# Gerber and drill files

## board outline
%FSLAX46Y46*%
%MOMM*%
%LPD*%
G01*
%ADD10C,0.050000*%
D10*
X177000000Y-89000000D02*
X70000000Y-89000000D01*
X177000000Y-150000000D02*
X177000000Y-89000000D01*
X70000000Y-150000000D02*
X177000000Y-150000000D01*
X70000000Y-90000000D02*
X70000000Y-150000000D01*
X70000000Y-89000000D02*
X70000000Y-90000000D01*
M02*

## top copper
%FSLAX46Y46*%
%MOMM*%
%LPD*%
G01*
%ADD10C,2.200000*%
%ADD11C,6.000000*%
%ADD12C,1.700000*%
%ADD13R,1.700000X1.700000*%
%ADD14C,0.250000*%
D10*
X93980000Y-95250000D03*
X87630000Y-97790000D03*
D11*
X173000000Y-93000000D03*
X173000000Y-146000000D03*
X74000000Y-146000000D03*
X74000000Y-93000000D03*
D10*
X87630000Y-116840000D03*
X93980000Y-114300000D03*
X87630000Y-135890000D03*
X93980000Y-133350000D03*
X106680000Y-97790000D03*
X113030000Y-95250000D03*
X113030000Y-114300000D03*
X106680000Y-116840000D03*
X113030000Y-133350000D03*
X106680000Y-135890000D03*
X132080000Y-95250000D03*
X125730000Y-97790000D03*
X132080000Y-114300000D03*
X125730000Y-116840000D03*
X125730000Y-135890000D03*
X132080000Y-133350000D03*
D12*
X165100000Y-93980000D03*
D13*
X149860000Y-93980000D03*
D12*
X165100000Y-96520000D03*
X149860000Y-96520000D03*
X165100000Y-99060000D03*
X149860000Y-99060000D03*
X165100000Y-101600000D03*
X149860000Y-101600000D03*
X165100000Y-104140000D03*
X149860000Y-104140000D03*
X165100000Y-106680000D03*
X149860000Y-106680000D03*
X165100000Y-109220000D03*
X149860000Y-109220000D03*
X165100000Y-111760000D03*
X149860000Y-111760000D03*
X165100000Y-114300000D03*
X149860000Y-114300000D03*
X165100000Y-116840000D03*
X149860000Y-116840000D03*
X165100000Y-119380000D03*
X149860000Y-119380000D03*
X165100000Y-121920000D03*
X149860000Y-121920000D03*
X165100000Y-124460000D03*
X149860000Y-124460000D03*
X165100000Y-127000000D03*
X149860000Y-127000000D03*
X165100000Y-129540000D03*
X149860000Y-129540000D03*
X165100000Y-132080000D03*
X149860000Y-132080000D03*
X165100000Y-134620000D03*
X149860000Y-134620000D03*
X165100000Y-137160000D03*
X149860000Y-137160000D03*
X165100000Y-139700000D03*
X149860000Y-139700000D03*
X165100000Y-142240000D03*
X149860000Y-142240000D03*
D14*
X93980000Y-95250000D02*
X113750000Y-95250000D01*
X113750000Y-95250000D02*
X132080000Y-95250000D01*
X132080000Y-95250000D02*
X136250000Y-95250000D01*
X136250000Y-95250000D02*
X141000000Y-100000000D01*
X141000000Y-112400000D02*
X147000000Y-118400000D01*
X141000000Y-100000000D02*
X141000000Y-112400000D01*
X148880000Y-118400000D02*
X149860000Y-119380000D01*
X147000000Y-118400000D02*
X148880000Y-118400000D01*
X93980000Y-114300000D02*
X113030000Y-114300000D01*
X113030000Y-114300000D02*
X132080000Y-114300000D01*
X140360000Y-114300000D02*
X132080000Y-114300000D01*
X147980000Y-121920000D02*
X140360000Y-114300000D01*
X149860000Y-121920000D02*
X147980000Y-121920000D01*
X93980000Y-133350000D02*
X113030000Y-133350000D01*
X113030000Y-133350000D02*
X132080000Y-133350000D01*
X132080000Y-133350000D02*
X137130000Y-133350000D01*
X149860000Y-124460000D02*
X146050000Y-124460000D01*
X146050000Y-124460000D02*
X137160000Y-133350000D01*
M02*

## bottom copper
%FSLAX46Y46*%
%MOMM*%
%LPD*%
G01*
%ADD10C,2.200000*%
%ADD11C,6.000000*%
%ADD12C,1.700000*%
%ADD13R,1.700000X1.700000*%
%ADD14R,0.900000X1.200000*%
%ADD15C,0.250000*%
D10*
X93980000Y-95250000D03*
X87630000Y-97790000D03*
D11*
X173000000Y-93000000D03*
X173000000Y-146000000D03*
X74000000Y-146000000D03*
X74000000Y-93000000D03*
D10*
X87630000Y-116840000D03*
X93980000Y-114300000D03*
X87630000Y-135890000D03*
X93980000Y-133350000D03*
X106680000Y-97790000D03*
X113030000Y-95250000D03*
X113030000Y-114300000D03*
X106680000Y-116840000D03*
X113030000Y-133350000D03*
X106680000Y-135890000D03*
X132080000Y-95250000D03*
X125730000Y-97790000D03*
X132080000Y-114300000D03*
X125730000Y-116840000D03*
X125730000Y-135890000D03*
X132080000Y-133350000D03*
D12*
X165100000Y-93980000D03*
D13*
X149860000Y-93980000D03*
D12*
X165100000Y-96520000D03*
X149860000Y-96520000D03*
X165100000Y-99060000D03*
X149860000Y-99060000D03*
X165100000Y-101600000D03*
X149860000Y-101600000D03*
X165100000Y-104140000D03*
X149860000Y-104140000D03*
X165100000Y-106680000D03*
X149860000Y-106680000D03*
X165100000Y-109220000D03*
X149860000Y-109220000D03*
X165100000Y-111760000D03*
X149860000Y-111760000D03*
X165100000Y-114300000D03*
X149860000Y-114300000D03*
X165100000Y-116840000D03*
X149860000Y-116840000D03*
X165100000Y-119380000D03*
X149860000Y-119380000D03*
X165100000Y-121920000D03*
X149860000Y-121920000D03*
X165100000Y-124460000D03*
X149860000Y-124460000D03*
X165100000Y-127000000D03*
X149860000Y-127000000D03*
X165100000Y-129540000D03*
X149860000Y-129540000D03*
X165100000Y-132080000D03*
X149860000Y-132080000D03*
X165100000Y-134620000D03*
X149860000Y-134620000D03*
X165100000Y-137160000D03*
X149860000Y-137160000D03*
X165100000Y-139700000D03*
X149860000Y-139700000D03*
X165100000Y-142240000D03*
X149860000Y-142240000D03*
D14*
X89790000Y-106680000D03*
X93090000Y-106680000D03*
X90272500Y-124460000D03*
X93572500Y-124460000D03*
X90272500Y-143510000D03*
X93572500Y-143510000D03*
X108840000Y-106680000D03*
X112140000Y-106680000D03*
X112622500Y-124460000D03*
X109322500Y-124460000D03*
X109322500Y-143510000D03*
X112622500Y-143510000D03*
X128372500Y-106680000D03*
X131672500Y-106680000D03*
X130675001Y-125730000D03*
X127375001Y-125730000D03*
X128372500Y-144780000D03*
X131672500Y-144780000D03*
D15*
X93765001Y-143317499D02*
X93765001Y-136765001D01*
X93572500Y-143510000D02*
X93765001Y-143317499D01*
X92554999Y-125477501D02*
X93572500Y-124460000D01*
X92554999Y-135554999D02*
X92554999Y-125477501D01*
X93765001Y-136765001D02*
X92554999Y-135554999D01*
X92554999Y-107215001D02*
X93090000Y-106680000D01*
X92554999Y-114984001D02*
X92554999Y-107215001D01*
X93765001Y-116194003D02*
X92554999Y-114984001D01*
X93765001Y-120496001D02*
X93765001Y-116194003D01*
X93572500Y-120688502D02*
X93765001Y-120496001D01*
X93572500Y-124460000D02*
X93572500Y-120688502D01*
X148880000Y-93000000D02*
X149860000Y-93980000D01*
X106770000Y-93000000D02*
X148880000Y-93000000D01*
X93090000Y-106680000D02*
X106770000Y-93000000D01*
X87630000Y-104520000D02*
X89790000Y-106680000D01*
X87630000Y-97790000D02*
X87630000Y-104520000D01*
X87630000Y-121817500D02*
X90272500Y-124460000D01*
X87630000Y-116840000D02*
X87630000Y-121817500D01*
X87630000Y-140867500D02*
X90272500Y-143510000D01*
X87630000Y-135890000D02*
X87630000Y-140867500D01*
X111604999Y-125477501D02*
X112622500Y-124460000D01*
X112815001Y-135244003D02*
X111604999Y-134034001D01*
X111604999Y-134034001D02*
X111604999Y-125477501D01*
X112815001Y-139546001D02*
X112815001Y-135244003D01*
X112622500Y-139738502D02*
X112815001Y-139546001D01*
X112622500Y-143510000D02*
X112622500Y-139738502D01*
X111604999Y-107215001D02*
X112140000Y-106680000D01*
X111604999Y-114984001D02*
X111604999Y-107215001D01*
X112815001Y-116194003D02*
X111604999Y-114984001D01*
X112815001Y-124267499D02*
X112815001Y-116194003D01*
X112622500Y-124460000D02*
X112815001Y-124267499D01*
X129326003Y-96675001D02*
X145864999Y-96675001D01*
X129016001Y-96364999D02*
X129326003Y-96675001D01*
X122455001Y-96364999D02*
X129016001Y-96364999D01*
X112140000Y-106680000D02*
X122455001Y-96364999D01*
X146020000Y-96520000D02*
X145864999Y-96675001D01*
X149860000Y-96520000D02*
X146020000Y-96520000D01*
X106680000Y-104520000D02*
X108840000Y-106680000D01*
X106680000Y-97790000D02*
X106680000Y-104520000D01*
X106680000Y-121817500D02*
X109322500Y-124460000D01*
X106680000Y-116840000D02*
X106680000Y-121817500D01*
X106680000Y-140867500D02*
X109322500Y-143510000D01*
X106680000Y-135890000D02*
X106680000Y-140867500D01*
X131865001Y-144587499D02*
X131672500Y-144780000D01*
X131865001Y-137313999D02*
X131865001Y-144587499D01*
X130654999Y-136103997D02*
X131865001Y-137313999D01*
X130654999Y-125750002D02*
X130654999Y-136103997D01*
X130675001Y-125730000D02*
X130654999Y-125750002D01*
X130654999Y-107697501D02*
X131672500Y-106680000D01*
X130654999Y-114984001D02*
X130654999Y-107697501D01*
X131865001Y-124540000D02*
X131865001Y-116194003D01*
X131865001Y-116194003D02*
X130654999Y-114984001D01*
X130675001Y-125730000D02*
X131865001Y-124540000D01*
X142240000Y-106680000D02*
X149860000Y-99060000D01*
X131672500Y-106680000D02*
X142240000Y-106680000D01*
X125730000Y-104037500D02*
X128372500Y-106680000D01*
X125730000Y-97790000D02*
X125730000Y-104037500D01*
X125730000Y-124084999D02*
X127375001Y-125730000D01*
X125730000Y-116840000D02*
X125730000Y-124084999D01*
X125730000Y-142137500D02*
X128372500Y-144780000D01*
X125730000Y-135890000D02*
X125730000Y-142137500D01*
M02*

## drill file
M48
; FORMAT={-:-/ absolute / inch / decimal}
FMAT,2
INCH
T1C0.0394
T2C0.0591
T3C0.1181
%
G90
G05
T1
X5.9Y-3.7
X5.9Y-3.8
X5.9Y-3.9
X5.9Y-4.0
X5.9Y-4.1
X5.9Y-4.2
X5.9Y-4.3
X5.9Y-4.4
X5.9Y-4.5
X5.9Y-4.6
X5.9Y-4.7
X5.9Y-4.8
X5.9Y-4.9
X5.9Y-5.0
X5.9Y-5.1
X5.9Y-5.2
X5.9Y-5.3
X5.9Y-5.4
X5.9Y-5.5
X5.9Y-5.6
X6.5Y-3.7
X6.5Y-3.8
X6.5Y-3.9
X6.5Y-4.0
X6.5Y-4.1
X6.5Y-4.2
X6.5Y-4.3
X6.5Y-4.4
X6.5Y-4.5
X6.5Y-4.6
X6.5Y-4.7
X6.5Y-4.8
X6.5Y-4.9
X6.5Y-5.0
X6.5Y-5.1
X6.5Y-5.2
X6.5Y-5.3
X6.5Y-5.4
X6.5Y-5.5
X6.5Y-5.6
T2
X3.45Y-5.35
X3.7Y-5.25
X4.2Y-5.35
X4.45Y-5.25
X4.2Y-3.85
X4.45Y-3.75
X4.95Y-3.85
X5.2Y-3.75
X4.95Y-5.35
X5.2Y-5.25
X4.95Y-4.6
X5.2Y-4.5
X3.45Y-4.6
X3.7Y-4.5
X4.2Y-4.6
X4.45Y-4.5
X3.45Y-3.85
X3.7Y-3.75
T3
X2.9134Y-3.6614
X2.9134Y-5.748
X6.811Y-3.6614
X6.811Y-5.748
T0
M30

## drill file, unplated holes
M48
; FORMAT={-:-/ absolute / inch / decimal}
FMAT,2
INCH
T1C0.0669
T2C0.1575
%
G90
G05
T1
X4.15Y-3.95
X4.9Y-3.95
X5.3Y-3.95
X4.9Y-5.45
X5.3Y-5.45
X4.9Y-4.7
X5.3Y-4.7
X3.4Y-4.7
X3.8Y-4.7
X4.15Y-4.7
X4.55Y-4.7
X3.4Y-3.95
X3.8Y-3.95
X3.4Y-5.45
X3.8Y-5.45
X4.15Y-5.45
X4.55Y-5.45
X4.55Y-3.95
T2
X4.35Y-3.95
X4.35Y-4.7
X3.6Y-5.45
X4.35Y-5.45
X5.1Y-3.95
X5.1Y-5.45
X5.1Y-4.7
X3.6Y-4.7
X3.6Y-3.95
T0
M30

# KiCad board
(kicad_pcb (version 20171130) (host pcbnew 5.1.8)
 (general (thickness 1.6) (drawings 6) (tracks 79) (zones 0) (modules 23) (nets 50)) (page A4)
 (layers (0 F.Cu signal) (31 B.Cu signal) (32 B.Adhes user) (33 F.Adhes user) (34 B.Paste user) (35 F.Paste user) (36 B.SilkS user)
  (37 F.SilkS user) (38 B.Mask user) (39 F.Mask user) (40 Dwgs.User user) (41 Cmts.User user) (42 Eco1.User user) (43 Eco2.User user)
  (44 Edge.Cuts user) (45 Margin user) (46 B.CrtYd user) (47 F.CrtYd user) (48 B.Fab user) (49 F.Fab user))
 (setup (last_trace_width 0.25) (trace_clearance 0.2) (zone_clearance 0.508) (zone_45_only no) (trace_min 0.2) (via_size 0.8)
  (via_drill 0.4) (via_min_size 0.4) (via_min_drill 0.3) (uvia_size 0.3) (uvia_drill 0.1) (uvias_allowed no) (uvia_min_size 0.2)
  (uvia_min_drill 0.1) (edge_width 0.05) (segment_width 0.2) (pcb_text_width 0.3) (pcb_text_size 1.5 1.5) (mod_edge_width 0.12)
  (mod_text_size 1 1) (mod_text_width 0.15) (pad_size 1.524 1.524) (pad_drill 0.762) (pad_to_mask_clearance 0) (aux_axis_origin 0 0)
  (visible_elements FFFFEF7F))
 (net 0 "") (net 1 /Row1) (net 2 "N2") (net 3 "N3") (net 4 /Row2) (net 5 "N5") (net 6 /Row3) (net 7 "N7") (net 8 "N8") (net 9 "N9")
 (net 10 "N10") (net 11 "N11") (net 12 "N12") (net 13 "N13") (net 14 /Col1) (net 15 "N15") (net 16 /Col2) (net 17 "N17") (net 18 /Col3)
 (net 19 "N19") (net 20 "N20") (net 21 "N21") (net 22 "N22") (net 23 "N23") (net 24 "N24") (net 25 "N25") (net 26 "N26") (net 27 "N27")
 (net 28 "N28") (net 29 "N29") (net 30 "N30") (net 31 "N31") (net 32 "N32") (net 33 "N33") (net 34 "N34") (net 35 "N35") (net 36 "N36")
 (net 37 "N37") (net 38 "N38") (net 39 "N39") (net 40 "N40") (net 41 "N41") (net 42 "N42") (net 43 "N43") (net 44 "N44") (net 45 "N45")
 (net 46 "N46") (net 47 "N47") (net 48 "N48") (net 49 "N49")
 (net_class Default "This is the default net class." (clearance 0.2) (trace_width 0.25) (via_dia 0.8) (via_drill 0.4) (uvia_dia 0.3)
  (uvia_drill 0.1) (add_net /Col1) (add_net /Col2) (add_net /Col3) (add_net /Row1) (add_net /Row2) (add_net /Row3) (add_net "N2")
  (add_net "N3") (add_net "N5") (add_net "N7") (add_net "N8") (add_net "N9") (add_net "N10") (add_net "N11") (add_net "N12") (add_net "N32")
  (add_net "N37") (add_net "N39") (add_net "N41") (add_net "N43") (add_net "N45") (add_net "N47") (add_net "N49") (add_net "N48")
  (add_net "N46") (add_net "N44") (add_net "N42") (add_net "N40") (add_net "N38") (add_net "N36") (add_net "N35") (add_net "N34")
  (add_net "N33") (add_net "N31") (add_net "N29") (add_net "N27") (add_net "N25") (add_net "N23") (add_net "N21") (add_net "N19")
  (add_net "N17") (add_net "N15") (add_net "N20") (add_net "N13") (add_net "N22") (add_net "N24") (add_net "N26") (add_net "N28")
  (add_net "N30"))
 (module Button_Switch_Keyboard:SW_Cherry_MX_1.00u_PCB (layer F.Cu) (at 93.98 95.25)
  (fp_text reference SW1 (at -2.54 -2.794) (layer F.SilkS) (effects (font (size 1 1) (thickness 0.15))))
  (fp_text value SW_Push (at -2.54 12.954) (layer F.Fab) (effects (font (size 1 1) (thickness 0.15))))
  (pad 1 thru_hole circle (at 0 0) (size 2.2 2.2) (drill 1.5) (layers *.Cu *.Mask) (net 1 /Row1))
  (pad 2 thru_hole circle (at -6.35 2.54) (size 2.2 2.2) (drill 1.5) (layers *.Cu *.Mask) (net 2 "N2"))
  (pad "" np_thru_hole circle (at -2.54 5.08) (size 4 4) (drill 4) (layers *.Cu *.Mask))
  (pad "" np_thru_hole circle (at -7.62 5.08) (size 1.7 1.7) (drill 1.7) (layers *.Cu *.Mask))
  (pad "" np_thru_hole circle (at 2.54 5.08) (size 1.7 1.7) (drill 1.7) (layers *.Cu *.Mask)))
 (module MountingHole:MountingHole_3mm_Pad (layer F.Cu) (at 173 93)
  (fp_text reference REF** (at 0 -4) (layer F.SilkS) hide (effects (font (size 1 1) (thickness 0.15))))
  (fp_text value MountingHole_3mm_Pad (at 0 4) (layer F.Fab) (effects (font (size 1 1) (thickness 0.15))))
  (pad 1 thru_hole circle (at 0 0) (size 6 6) (drill 3) (layers *.Cu *.Mask)))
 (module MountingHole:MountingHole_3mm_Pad (layer F.Cu) (at 173 146)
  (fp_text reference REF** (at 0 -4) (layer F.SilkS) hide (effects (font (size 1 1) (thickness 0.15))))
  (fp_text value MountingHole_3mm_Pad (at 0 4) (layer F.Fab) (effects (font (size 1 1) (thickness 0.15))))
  (pad 1 thru_hole circle (at 0 0) (size 6 6) (drill 3) (layers *.Cu *.Mask)))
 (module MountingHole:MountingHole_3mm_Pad (layer F.Cu) (at 74 146)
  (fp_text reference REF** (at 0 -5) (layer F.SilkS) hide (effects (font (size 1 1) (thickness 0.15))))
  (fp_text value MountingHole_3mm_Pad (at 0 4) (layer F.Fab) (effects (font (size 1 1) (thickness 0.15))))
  (pad 1 thru_hole circle (at 0 0) (size 6 6) (drill 3) (layers *.Cu *.Mask)))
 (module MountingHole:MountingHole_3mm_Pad (layer F.Cu) (at 74 93)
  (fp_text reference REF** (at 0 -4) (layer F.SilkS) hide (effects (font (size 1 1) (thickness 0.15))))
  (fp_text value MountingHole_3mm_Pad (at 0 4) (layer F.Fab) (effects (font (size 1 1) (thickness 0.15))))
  (pad 1 thru_hole circle (at 0 0) (size 6 6) (drill 3) (layers *.Cu *.Mask)))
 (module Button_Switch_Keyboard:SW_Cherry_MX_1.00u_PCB (layer F.Cu) (at 93.98 114.3)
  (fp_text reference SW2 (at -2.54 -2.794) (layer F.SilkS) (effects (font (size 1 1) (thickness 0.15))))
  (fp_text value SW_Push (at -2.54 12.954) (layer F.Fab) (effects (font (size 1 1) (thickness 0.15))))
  (pad "" np_thru_hole circle (at 2.54 5.08) (size 1.7 1.7) (drill 1.7) (layers *.Cu *.Mask))
  (pad "" np_thru_hole circle (at -7.62 5.08) (size 1.7 1.7) (drill 1.7) (layers *.Cu *.Mask))
  (pad "" np_thru_hole circle (at -2.54 5.08) (size 4 4) (drill 4) (layers *.Cu *.Mask))
  (pad 2 thru_hole circle (at -6.35 2.54) (size 2.2 2.2) (drill 1.5) (layers *.Cu *.Mask) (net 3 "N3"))
  (pad 1 thru_hole circle (at 0 0) (size 2.2 2.2) (drill 1.5) (layers *.Cu *.Mask) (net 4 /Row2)))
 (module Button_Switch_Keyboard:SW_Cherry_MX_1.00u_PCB (layer F.Cu) (at 93.98 133.35)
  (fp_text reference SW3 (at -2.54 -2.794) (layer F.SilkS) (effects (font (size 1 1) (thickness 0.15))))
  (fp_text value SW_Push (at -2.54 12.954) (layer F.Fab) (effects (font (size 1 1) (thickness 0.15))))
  (pad "" np_thru_hole circle (at 2.54 5.08) (size 1.7 1.7) (drill 1.7) (layers *.Cu *.Mask))
  (pad "" np_thru_hole circle (at -7.62 5.08) (size 1.7 1.7) (drill 1.7) (layers *.Cu *.Mask))
  (pad "" np_thru_hole circle (at -2.54 5.08) (size 4 4) (drill 4) (layers *.Cu *.Mask))
  (pad 2 thru_hole circle (at -6.35 2.54) (size 2.2 2.2) (drill 1.5) (layers *.Cu *.Mask) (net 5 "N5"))
  (pad 1 thru_hole circle (at 0 0) (size 2.2 2.2) (drill 1.5) (layers *.Cu *.Mask) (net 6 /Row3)))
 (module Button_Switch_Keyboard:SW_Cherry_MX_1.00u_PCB (layer F.Cu) (at 113.03 95.25)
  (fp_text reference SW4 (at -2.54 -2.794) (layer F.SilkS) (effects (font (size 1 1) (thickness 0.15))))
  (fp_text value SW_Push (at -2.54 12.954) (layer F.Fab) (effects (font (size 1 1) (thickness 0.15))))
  (pad "" np_thru_hole circle (at 2.54 5.08) (size 1.7 1.7) (drill 1.7) (layers *.Cu *.Mask))
  (pad "" np_thru_hole circle (at -7.62 5.08) (size 1.7 1.7) (drill 1.7) (layers *.Cu *.Mask))
  (pad "" np_thru_hole circle (at -2.54 5.08) (size 4 4) (drill 4) (layers *.Cu *.Mask))
  (pad 2 thru_hole circle (at -6.35 2.54) (size 2.2 2.2) (drill 1.5) (layers *.Cu *.Mask) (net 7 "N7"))
  (pad 1 thru_hole circle (at 0 0) (size 2.2 2.2) (drill 1.5) (layers *.Cu *.Mask) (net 1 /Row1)))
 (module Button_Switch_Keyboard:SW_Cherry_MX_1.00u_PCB (layer F.Cu) (at 113.03 114.3)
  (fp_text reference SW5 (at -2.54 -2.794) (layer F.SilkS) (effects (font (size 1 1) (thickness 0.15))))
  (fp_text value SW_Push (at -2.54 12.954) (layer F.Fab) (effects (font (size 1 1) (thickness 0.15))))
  (pad 1 thru_hole circle (at 0 0) (size 2.2 2.2) (drill 1.5) (layers *.Cu *.Mask) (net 4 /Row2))
  (pad 2 thru_hole circle (at -6.35 2.54) (size 2.2 2.2) (drill 1.5) (layers *.Cu *.Mask) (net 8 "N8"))
  (pad "" np_thru_hole circle (at -2.54 5.08) (size 4 4) (drill 4) (layers *.Cu *.Mask))
  (pad "" np_thru_hole circle (at -7.62 5.08) (size 1.7 1.7) (drill 1.7) (layers *.Cu *.Mask))
  (pad "" np_thru_hole circle (at 2.54 5.08) (size 1.7 1.7) (drill 1.7) (layers *.Cu *.Mask)))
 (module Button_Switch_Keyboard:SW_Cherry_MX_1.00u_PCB (layer F.Cu) (at 113.03 133.35)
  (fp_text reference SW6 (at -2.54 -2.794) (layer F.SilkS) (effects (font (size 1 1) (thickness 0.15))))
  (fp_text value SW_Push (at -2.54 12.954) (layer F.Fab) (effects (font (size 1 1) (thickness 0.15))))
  (pad 1 thru_hole circle (at 0 0) (size 2.2 2.2) (drill 1.5) (layers *.Cu *.Mask) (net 6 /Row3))
  (pad 2 thru_hole circle (at -6.35 2.54) (size 2.2 2.2) (drill 1.5) (layers *.Cu *.Mask) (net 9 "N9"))
  (pad "" np_thru_hole circle (at -2.54 5.08) (size 4 4) (drill 4) (layers *.Cu *.Mask))
  (pad "" np_thru_hole circle (at -7.62 5.08) (size 1.7 1.7) (drill 1.7) (layers *.Cu *.Mask))
  (pad "" np_thru_hole circle (at 2.54 5.08) (size 1.7 1.7) (drill 1.7) (layers *.Cu *.Mask)))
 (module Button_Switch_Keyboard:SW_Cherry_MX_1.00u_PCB (layer F.Cu) (at 132.08 95.25)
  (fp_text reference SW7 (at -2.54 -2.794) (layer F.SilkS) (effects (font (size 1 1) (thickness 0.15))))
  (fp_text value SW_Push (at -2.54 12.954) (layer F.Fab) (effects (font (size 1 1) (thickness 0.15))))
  (pad 1 thru_hole circle (at 0 0) (size 2.2 2.2) (drill 1.5) (layers *.Cu *.Mask) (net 1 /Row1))
  (pad 2 thru_hole circle (at -6.35 2.54) (size 2.2 2.2) (drill 1.5) (layers *.Cu *.Mask) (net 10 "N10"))
  (pad "" np_thru_hole circle (at -2.54 5.08) (size 4 4) (drill 4) (layers *.Cu *.Mask))
  (pad "" np_thru_hole circle (at -7.62 5.08) (size 1.7 1.7) (drill 1.7) (layers *.Cu *.Mask))
  (pad "" np_thru_hole circle (at 2.54 5.08) (size 1.7 1.7) (drill 1.7) (layers *.Cu *.Mask)))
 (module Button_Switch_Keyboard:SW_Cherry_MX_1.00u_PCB (layer F.Cu) (at 132.08 114.3)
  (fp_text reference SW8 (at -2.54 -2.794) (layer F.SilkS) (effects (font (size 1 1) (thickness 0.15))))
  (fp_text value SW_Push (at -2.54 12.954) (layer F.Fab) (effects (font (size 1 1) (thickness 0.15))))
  (pad 1 thru_hole circle (at 0 0) (size 2.2 2.2) (drill 1.5) (layers *.Cu *.Mask) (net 4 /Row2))
  (pad 2 thru_hole circle (at -6.35 2.54) (size 2.2 2.2) (drill 1.5) (layers *.Cu *.Mask) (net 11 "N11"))
  (pad "" np_thru_hole circle (at -2.54 5.08) (size 4 4) (drill 4) (layers *.Cu *.Mask))
  (pad "" np_thru_hole circle (at -7.62 5.08) (size 1.7 1.7) (drill 1.7) (layers *.Cu *.Mask))
  (pad "" np_thru_hole circle (at 2.54 5.08) (size 1.7 1.7) (drill 1.7) (layers *.Cu *.Mask)))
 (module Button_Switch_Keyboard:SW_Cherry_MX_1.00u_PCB (layer F.Cu) (at 132.08 133.35)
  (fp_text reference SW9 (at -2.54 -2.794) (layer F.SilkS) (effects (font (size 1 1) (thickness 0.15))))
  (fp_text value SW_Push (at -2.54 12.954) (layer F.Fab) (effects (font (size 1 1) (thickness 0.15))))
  (pad "" np_thru_hole circle (at 2.54 5.08) (size 1.7 1.7) (drill 1.7) (layers *.Cu *.Mask))
  (pad "" np_thru_hole circle (at -7.62 5.08) (size 1.7 1.7) (drill 1.7) (layers *.Cu *.Mask))
  (pad "" np_thru_hole circle (at -2.54 5.08) (size 4 4) (drill 4) (layers *.Cu *.Mask))
  (pad 2 thru_hole circle (at -6.35 2.54) (size 2.2 2.2) (drill 1.5) (layers *.Cu *.Mask) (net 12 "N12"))
  (pad 1 thru_hole circle (at 0 0) (size 2.2 2.2) (drill 1.5) (layers *.Cu *.Mask) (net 6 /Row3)))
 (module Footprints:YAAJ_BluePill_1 (layer F.Cu) (at 149.86 93.98)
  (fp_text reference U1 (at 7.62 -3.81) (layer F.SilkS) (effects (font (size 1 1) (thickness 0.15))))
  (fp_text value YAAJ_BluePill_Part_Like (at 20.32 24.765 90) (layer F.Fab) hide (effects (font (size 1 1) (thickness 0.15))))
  (pad 40 thru_hole circle (at 15.24 0) (size 1.7 1.7) (drill 1) (layers *.Cu *.Mask) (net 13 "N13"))
  (pad 1 thru_hole rect (at 0 0) (size 1.7 1.7) (drill 1) (layers *.Cu *.Mask) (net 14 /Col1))
  (pad 39 thru_hole circle (at 15.24 2.54) (size 1.7 1.7) (drill 1) (layers *.Cu *.Mask) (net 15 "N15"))
  (pad 2 thru_hole circle (at 0 2.54) (size 1.7 1.7) (drill 1) (layers *.Cu *.Mask) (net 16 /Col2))
  (pad 38 thru_hole circle (at 15.24 5.08) (size 1.7 1.7) (drill 1) (layers *.Cu *.Mask) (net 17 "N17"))
  (pad 3 thru_hole circle (at 0 5.08) (size 1.7 1.7) (drill 1) (layers *.Cu *.Mask) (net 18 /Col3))
  (pad 37 thru_hole circle (at 15.24 7.62) (size 1.7 1.7) (drill 1) (layers *.Cu *.Mask) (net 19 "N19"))
  (pad 4 thru_hole circle (at 0 7.62) (size 1.7 1.7) (drill 1) (layers *.Cu *.Mask) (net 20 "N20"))
  (pad 36 thru_hole circle (at 15.24 10.16) (size 1.7 1.7) (drill 1) (layers *.Cu *.Mask) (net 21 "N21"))
  (pad 5 thru_hole circle (at 0 10.16) (size 1.7 1.7) (drill 1) (layers *.Cu *.Mask) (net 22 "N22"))
  (pad 35 thru_hole circle (at 15.24 12.7) (size 1.7 1.7) (drill 1) (layers *.Cu *.Mask) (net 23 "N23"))
  (pad 6 thru_hole circle (at 0 12.7) (size 1.7 1.7) (drill 1) (layers *.Cu *.Mask) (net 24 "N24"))
  (pad 34 thru_hole circle (at 15.24 15.24) (size 1.7 1.7) (drill 1) (layers *.Cu *.Mask) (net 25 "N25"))
  (pad 7 thru_hole circle (at 0 15.24) (size 1.7 1.7) (drill 1) (layers *.Cu *.Mask) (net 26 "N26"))
  (pad 33 thru_hole circle (at 15.24 17.78) (size 1.7 1.7) (drill 1) (layers *.Cu *.Mask) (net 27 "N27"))
  (pad 8 thru_hole circle (at 0 17.78) (size 1.7 1.7) (drill 1) (layers *.Cu *.Mask) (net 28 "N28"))
  (pad 32 thru_hole circle (at 15.24 20.32) (size 1.7 1.7) (drill 1) (layers *.Cu *.Mask) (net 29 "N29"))
  (pad 9 thru_hole circle (at 0 20.32) (size 1.7 1.7) (drill 1) (layers *.Cu *.Mask) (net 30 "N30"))
  (pad 31 thru_hole circle (at 15.24 22.86) (size 1.7 1.7) (drill 1) (layers *.Cu *.Mask) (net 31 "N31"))
  (pad 10 thru_hole circle (at 0 22.86) (size 1.7 1.7) (drill 1) (layers *.Cu *.Mask) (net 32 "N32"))
  (pad 30 thru_hole circle (at 15.24 25.4) (size 1.7 1.7) (drill 1) (layers *.Cu *.Mask) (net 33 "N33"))
  (pad 11 thru_hole circle (at 0 25.4) (size 1.7 1.7) (drill 1) (layers *.Cu *.Mask) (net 1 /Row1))
  (pad 29 thru_hole circle (at 15.24 27.94) (size 1.7 1.7) (drill 1) (layers *.Cu *.Mask) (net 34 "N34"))
  (pad 12 thru_hole circle (at 0 27.94) (size 1.7 1.7) (drill 1) (layers *.Cu *.Mask) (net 4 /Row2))
  (pad 28 thru_hole circle (at 15.24 30.48) (size 1.7 1.7) (drill 1) (layers *.Cu *.Mask) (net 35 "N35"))
  (pad 13 thru_hole circle (at 0 30.48) (size 1.7 1.7) (drill 1) (layers *.Cu *.Mask) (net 6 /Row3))
  (pad 27 thru_hole circle (at 15.24 33.02) (size 1.7 1.7) (drill 1) (layers *.Cu *.Mask) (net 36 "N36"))
  (pad 14 thru_hole circle (at 0 33.02) (size 1.7 1.7) (drill 1) (layers *.Cu *.Mask) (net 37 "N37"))
  (pad 26 thru_hole circle (at 15.24 35.56) (size 1.7 1.7) (drill 1) (layers *.Cu *.Mask) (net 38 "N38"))
  (pad 15 thru_hole circle (at 0 35.56) (size 1.7 1.7) (drill 1) (layers *.Cu *.Mask) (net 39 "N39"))
  (pad 25 thru_hole circle (at 15.24 38.1) (size 1.7 1.7) (drill 1) (layers *.Cu *.Mask) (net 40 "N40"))
  (pad 16 thru_hole circle (at 0 38.1) (size 1.7 1.7) (drill 1) (layers *.Cu *.Mask) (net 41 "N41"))
  (pad 24 thru_hole circle (at 15.24 40.64) (size 1.7 1.7) (drill 1) (layers *.Cu *.Mask) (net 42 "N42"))
  (pad 17 thru_hole circle (at 0 40.64) (size 1.7 1.7) (drill 1) (layers *.Cu *.Mask) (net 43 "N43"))
  (pad 23 thru_hole circle (at 15.24 43.18) (size 1.7 1.7) (drill 1) (layers *.Cu *.Mask) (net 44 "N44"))
  (pad 18 thru_hole circle (at 0 43.18) (size 1.7 1.7) (drill 1) (layers *.Cu *.Mask) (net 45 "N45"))
  (pad 22 thru_hole circle (at 15.24 45.72) (size 1.7 1.7) (drill 1) (layers *.Cu *.Mask) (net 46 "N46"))
  (pad 19 thru_hole circle (at 0 45.72) (size 1.7 1.7) (drill 1) (layers *.Cu *.Mask) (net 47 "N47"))
  (pad 21 thru_hole circle (at 15.24 48.26) (size 1.7 1.7) (drill 1) (layers *.Cu *.Mask) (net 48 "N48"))
  (pad 20 thru_hole circle (at 0 48.26) (size 1.7 1.7) (drill 1) (layers *.Cu *.Mask) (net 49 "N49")))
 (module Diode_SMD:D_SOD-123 (layer B.Cu) (at 91.44 106.68)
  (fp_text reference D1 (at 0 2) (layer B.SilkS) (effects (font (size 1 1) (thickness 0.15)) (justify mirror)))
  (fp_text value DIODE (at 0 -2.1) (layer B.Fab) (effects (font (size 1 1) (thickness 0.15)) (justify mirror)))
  (pad 1 smd rect (at -1.65 0) (size 0.9 1.2) (layers B.Cu B.Paste B.Mask) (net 2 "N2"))
  (pad 2 smd rect (at 1.65 0) (size 0.9 1.2) (layers B.Cu B.Paste B.Mask) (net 14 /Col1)))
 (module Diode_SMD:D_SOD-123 (layer B.Cu) (at 91.9225 124.46)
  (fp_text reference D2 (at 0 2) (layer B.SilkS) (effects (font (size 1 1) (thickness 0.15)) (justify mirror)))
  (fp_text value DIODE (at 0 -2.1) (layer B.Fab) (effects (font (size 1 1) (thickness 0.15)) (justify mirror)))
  (pad 1 smd rect (at -1.65 0) (size 0.9 1.2) (layers B.Cu B.Paste B.Mask) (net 3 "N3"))
  (pad 2 smd rect (at 1.65 0) (size 0.9 1.2) (layers B.Cu B.Paste B.Mask) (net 14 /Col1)))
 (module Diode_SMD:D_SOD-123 (layer B.Cu) (at 91.9225 143.51)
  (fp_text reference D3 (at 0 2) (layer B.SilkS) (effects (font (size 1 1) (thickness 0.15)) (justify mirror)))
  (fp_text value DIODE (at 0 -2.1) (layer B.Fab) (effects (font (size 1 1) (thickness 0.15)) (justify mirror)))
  (pad 1 smd rect (at -1.65 0) (size 0.9 1.2) (layers B.Cu B.Paste B.Mask) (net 5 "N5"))
  (pad 2 smd rect (at 1.65 0) (size 0.9 1.2) (layers B.Cu B.Paste B.Mask) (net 14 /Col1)))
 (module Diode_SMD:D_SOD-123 (layer B.Cu) (at 110.49 106.68)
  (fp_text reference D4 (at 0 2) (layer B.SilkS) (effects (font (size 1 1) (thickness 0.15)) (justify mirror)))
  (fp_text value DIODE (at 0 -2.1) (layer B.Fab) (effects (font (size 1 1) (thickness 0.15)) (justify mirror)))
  (pad 1 smd rect (at -1.65 0) (size 0.9 1.2) (layers B.Cu B.Paste B.Mask) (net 7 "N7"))
  (pad 2 smd rect (at 1.65 0) (size 0.9 1.2) (layers B.Cu B.Paste B.Mask) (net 16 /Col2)))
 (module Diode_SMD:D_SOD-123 (layer B.Cu) (at 110.9725 124.46)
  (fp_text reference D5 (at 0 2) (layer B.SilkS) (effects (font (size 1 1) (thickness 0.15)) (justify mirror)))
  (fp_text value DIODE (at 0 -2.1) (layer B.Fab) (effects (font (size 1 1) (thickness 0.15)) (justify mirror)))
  (pad 2 smd rect (at 1.65 0) (size 0.9 1.2) (layers B.Cu B.Paste B.Mask) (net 16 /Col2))
  (pad 1 smd rect (at -1.65 0) (size 0.9 1.2) (layers B.Cu B.Paste B.Mask) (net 8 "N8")))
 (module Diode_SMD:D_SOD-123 (layer B.Cu) (at 110.9725 143.51)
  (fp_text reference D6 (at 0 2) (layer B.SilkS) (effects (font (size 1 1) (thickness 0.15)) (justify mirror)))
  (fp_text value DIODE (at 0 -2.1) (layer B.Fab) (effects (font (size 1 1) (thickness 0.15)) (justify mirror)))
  (pad 1 smd rect (at -1.65 0) (size 0.9 1.2) (layers B.Cu B.Paste B.Mask) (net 9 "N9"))
  (pad 2 smd rect (at 1.65 0) (size 0.9 1.2) (layers B.Cu B.Paste B.Mask) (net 16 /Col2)))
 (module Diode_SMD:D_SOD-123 (layer B.Cu) (at 130.0225 106.68)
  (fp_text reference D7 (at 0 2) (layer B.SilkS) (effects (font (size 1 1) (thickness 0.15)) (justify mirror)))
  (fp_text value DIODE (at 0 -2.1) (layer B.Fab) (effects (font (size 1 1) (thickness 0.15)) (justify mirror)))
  (pad 1 smd rect (at -1.65 0) (size 0.9 1.2) (layers B.Cu B.Paste B.Mask) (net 10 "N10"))
  (pad 2 smd rect (at 1.65 0) (size 0.9 1.2) (layers B.Cu B.Paste B.Mask) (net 18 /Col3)))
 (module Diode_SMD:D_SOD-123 (layer B.Cu) (at 129.025001 125.73)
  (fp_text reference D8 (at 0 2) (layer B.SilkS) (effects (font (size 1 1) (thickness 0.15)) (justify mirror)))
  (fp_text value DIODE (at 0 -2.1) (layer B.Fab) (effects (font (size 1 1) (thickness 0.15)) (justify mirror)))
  (pad 2 smd rect (at 1.65 0) (size 0.9 1.2) (layers B.Cu B.Paste B.Mask) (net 18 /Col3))
  (pad 1 smd rect (at -1.65 0) (size 0.9 1.2) (layers B.Cu B.Paste B.Mask) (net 11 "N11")))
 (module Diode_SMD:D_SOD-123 (layer B.Cu) (at 130.0225 144.78)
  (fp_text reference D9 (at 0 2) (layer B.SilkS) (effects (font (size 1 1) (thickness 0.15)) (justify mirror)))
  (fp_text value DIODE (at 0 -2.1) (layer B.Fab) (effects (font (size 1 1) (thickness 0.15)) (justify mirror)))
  (pad 1 smd rect (at -1.65 0) (size 0.9 1.2) (layers B.Cu B.Paste B.Mask) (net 12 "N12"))
  (pad 2 smd rect (at 1.65 0) (size 0.9 1.2) (layers B.Cu B.Paste B.Mask) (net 18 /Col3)))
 (gr_line (start 177 89) (end 70 89) (layer Edge.Cuts) (width 0.05))
 (gr_line (start 177 150) (end 177 89) (layer Edge.Cuts) (width 0.05))
 (gr_line (start 70 150) (end 177 150) (layer Edge.Cuts) (width 0.05))
 (gr_line (start 70 90) (end 70 150) (layer Edge.Cuts) (width 0.05))
 (gr_line (start 70 89) (end 70 90) (layer Edge.Cuts) (width 0.05))
 (segment (start 93.765001 143.317499) (end 93.765001 136.765001) (width 0.25) (layer B.Cu) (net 14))
 (segment (start 93.5725 143.51) (end 93.765001 143.317499) (width 0.25) (layer B.Cu) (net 14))
 (segment (start 92.554999 125.477501) (end 93.5725 124.46) (width 0.25) (layer B.Cu) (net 14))
 (segment (start 92.554999 135.554999) (end 92.554999 125.477501) (width 0.25) (layer B.Cu) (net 14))
 (segment (start 93.765001 136.765001) (end 92.554999 135.554999) (width 0.25) (layer B.Cu) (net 14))
 (segment (start 92.554999 107.215001) (end 93.09 106.68) (width 0.25) (layer B.Cu) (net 14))
 (segment (start 92.554999 114.984001) (end 92.554999 107.215001) (width 0.25) (layer B.Cu) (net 14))
 (segment (start 93.765001 116.194003) (end 92.554999 114.984001) (width 0.25) (layer B.Cu) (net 14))
 (segment (start 93.765001 120.496001) (end 93.765001 116.194003) (width 0.25) (layer B.Cu) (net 14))
 (segment (start 93.5725 120.688502) (end 93.765001 120.496001) (width 0.25) (layer B.Cu) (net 14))
 (segment (start 93.5725 124.46) (end 93.5725 120.688502) (width 0.25) (layer B.Cu) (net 14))
 (segment (start 148.88 93) (end 149.86 93.98) (width 0.25) (layer B.Cu) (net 14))
 (segment (start 106.77 93) (end 148.88 93) (width 0.25) (layer B.Cu) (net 14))
 (segment (start 93.09 106.68) (end 106.77 93) (width 0.25) (layer B.Cu) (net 14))
 (segment (start 87.63 104.52) (end 89.79 106.68) (width 0.25) (layer B.Cu) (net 2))
 (segment (start 87.63 97.79) (end 87.63 104.52) (width 0.25) (layer B.Cu) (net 2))
 (segment (start 87.63 121.8175) (end 90.2725 124.46) (width 0.25) (layer B.Cu) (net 3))
 (segment (start 87.63 116.84) (end 87.63 121.8175) (width 0.25) (layer B.Cu) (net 3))
 (segment (start 87.63 140.8675) (end 90.2725 143.51) (width 0.25) (layer B.Cu) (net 5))
 (segment (start 87.63 135.89) (end 87.63 140.8675) (width 0.25) (layer B.Cu) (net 5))
 (segment (start 111.604999 125.477501) (end 112.6225 124.46) (width 0.25) (layer B.Cu) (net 16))
 (segment (start 112.815001 135.244003) (end 111.604999 134.034001) (width 0.25) (layer B.Cu) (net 16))
 (segment (start 111.604999 134.034001) (end 111.604999 125.477501) (width 0.25) (layer B.Cu) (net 16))
 (segment (start 112.815001 139.546001) (end 112.815001 135.244003) (width 0.25) (layer B.Cu) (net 16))
 (segment (start 112.6225 139.738502) (end 112.815001 139.546001) (width 0.25) (layer B.Cu) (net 16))
 (segment (start 112.6225 143.51) (end 112.6225 139.738502) (width 0.25) (layer B.Cu) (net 16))
 (segment (start 111.604999 107.215001) (end 112.14 106.68) (width 0.25) (layer B.Cu) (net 16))
 (segment (start 111.604999 114.984001) (end 111.604999 107.215001) (width 0.25) (layer B.Cu) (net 16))
 (segment (start 112.815001 116.194003) (end 111.604999 114.984001) (width 0.25) (layer B.Cu) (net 16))
 (segment (start 112.815001 124.267499) (end 112.815001 116.194003) (width 0.25) (layer B.Cu) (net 16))
 (segment (start 112.6225 124.46) (end 112.815001 124.267499) (width 0.25) (layer B.Cu) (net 16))
 (segment (start 129.326003 96.675001) (end 145.864999 96.675001) (width 0.25) (layer B.Cu) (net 16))
 (segment (start 129.016001 96.364999) (end 129.326003 96.675001) (width 0.25) (layer B.Cu) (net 16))
 (segment (start 122.455001 96.364999) (end 129.016001 96.364999) (width 0.25) (layer B.Cu) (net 16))
 (segment (start 112.14 106.68) (end 122.455001 96.364999) (width 0.25) (layer B.Cu) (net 16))
 (segment (start 146.02 96.52) (end 145.864999 96.675001) (width 0.25) (layer B.Cu) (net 16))
 (segment (start 149.86 96.52) (end 146.02 96.52) (width 0.25) (layer B.Cu) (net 16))
 (segment (start 106.68 104.52) (end 108.84 106.68) (width 0.25) (layer B.Cu) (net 7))
 (segment (start 106.68 97.79) (end 106.68 104.52) (width 0.25) (layer B.Cu) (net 7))
 (segment (start 106.68 121.8175) (end 109.3225 124.46) (width 0.25) (layer B.Cu) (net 8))
 (segment (start 106.68 116.84) (end 106.68 121.8175) (width 0.25) (layer B.Cu) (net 8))
 (segment (start 106.68 140.8675) (end 109.3225 143.51) (width 0.25) (layer B.Cu) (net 9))
 (segment (start 106.68 135.89) (end 106.68 140.8675) (width 0.25) (layer B.Cu) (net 9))
 (segment (start 131.865001 144.587499) (end 131.6725 144.78) (width 0.25) (layer B.Cu) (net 18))
 (segment (start 131.865001 137.313999) (end 131.865001 144.587499) (width 0.25) (layer B.Cu) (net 18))
 (segment (start 130.654999 136.103997) (end 131.865001 137.313999) (width 0.25) (layer B.Cu) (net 18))
 (segment (start 130.654999 125.750002) (end 130.654999 136.103997) (width 0.25) (layer B.Cu) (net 18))
 (segment (start 130.675001 125.73) (end 130.654999 125.750002) (width 0.25) (layer B.Cu) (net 18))
 (segment (start 130.654999 107.697501) (end 131.6725 106.68) (width 0.25) (layer B.Cu) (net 18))
 (segment (start 130.654999 114.984001) (end 130.654999 107.697501) (width 0.25) (layer B.Cu) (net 18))
 (segment (start 131.865001 124.54) (end 131.865001 116.194003) (width 0.25) (layer B.Cu) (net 18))
 (segment (start 131.865001 116.194003) (end 130.654999 114.984001) (width 0.25) (layer B.Cu) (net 18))
 (segment (start 130.675001 125.73) (end 131.865001 124.54) (width 0.25) (layer B.Cu) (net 18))
 (segment (start 142.24 106.68) (end 149.86 99.06) (width 0.25) (layer B.Cu) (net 18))
 (segment (start 131.6725 106.68) (end 142.24 106.68) (width 0.25) (layer B.Cu) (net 18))
 (segment (start 125.73 104.0375) (end 128.3725 106.68) (width 0.25) (layer B.Cu) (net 10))
 (segment (start 125.73 97.79) (end 125.73 104.0375) (width 0.25) (layer B.Cu) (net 10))
 (segment (start 125.73 124.084999) (end 127.375001 125.73) (width 0.25) (layer B.Cu) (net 11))
 (segment (start 125.73 116.84) (end 125.73 124.084999) (width 0.25) (layer B.Cu) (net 11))
 (segment (start 125.73 142.1375) (end 128.3725 144.78) (width 0.25) (layer B.Cu) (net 12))
 (segment (start 125.73 135.89) (end 125.73 142.1375) (width 0.25) (layer B.Cu) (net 12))
 (segment (start 93.98 95.25) (end 113.75 95.25) (width 0.25) (layer F.Cu) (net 1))
 (segment (start 113.75 95.25) (end 132.08 95.25) (width 0.25) (layer F.Cu) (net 1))
 (segment (start 132.08 95.25) (end 136.25 95.25) (width 0.25) (layer F.Cu) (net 1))
 (segment (start 136.25 95.25) (end 141 100) (width 0.25) (layer F.Cu) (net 1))
 (segment (start 141 112.4) (end 147 118.4) (width 0.25) (layer F.Cu) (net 1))
 (segment (start 141 100) (end 141 112.4) (width 0.25) (layer F.Cu) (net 1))
 (segment (start 148.88 118.4) (end 149.86 119.38) (width 0.25) (layer F.Cu) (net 1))
 (segment (start 147 118.4) (end 148.88 118.4) (width 0.25) (layer F.Cu) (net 1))
 (segment (start 93.98 114.3) (end 113.03 114.3) (width 0.25) (layer F.Cu) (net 4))
 (segment (start 113.03 114.3) (end 132.08 114.3) (width 0.25) (layer F.Cu) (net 4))
 (segment (start 140.36 114.3) (end 132.08 114.3) (width 0.25) (layer F.Cu) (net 4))
 (segment (start 147.98 121.92) (end 140.36 114.3) (width 0.25) (layer F.Cu) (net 4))
 (segment (start 149.86 121.92) (end 147.98 121.92) (width 0.25) (layer F.Cu) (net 4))
 (segment (start 93.98 133.35) (end 113.03 133.35) (width 0.25) (layer F.Cu) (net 6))
 (segment (start 113.03 133.35) (end 132.08 133.35) (width 0.25) (layer F.Cu) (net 6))
 (segment (start 132.08 133.35) (end 137.13 133.35) (width 0.25) (layer F.Cu) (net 6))
 (segment (start 149.86 124.46) (end 146.05 124.46) (width 0.25) (layer F.Cu) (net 6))
 (segment (start 146.05 124.46) (end 137.16 133.35) (width 0.25) (layer F.Cu) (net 6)))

